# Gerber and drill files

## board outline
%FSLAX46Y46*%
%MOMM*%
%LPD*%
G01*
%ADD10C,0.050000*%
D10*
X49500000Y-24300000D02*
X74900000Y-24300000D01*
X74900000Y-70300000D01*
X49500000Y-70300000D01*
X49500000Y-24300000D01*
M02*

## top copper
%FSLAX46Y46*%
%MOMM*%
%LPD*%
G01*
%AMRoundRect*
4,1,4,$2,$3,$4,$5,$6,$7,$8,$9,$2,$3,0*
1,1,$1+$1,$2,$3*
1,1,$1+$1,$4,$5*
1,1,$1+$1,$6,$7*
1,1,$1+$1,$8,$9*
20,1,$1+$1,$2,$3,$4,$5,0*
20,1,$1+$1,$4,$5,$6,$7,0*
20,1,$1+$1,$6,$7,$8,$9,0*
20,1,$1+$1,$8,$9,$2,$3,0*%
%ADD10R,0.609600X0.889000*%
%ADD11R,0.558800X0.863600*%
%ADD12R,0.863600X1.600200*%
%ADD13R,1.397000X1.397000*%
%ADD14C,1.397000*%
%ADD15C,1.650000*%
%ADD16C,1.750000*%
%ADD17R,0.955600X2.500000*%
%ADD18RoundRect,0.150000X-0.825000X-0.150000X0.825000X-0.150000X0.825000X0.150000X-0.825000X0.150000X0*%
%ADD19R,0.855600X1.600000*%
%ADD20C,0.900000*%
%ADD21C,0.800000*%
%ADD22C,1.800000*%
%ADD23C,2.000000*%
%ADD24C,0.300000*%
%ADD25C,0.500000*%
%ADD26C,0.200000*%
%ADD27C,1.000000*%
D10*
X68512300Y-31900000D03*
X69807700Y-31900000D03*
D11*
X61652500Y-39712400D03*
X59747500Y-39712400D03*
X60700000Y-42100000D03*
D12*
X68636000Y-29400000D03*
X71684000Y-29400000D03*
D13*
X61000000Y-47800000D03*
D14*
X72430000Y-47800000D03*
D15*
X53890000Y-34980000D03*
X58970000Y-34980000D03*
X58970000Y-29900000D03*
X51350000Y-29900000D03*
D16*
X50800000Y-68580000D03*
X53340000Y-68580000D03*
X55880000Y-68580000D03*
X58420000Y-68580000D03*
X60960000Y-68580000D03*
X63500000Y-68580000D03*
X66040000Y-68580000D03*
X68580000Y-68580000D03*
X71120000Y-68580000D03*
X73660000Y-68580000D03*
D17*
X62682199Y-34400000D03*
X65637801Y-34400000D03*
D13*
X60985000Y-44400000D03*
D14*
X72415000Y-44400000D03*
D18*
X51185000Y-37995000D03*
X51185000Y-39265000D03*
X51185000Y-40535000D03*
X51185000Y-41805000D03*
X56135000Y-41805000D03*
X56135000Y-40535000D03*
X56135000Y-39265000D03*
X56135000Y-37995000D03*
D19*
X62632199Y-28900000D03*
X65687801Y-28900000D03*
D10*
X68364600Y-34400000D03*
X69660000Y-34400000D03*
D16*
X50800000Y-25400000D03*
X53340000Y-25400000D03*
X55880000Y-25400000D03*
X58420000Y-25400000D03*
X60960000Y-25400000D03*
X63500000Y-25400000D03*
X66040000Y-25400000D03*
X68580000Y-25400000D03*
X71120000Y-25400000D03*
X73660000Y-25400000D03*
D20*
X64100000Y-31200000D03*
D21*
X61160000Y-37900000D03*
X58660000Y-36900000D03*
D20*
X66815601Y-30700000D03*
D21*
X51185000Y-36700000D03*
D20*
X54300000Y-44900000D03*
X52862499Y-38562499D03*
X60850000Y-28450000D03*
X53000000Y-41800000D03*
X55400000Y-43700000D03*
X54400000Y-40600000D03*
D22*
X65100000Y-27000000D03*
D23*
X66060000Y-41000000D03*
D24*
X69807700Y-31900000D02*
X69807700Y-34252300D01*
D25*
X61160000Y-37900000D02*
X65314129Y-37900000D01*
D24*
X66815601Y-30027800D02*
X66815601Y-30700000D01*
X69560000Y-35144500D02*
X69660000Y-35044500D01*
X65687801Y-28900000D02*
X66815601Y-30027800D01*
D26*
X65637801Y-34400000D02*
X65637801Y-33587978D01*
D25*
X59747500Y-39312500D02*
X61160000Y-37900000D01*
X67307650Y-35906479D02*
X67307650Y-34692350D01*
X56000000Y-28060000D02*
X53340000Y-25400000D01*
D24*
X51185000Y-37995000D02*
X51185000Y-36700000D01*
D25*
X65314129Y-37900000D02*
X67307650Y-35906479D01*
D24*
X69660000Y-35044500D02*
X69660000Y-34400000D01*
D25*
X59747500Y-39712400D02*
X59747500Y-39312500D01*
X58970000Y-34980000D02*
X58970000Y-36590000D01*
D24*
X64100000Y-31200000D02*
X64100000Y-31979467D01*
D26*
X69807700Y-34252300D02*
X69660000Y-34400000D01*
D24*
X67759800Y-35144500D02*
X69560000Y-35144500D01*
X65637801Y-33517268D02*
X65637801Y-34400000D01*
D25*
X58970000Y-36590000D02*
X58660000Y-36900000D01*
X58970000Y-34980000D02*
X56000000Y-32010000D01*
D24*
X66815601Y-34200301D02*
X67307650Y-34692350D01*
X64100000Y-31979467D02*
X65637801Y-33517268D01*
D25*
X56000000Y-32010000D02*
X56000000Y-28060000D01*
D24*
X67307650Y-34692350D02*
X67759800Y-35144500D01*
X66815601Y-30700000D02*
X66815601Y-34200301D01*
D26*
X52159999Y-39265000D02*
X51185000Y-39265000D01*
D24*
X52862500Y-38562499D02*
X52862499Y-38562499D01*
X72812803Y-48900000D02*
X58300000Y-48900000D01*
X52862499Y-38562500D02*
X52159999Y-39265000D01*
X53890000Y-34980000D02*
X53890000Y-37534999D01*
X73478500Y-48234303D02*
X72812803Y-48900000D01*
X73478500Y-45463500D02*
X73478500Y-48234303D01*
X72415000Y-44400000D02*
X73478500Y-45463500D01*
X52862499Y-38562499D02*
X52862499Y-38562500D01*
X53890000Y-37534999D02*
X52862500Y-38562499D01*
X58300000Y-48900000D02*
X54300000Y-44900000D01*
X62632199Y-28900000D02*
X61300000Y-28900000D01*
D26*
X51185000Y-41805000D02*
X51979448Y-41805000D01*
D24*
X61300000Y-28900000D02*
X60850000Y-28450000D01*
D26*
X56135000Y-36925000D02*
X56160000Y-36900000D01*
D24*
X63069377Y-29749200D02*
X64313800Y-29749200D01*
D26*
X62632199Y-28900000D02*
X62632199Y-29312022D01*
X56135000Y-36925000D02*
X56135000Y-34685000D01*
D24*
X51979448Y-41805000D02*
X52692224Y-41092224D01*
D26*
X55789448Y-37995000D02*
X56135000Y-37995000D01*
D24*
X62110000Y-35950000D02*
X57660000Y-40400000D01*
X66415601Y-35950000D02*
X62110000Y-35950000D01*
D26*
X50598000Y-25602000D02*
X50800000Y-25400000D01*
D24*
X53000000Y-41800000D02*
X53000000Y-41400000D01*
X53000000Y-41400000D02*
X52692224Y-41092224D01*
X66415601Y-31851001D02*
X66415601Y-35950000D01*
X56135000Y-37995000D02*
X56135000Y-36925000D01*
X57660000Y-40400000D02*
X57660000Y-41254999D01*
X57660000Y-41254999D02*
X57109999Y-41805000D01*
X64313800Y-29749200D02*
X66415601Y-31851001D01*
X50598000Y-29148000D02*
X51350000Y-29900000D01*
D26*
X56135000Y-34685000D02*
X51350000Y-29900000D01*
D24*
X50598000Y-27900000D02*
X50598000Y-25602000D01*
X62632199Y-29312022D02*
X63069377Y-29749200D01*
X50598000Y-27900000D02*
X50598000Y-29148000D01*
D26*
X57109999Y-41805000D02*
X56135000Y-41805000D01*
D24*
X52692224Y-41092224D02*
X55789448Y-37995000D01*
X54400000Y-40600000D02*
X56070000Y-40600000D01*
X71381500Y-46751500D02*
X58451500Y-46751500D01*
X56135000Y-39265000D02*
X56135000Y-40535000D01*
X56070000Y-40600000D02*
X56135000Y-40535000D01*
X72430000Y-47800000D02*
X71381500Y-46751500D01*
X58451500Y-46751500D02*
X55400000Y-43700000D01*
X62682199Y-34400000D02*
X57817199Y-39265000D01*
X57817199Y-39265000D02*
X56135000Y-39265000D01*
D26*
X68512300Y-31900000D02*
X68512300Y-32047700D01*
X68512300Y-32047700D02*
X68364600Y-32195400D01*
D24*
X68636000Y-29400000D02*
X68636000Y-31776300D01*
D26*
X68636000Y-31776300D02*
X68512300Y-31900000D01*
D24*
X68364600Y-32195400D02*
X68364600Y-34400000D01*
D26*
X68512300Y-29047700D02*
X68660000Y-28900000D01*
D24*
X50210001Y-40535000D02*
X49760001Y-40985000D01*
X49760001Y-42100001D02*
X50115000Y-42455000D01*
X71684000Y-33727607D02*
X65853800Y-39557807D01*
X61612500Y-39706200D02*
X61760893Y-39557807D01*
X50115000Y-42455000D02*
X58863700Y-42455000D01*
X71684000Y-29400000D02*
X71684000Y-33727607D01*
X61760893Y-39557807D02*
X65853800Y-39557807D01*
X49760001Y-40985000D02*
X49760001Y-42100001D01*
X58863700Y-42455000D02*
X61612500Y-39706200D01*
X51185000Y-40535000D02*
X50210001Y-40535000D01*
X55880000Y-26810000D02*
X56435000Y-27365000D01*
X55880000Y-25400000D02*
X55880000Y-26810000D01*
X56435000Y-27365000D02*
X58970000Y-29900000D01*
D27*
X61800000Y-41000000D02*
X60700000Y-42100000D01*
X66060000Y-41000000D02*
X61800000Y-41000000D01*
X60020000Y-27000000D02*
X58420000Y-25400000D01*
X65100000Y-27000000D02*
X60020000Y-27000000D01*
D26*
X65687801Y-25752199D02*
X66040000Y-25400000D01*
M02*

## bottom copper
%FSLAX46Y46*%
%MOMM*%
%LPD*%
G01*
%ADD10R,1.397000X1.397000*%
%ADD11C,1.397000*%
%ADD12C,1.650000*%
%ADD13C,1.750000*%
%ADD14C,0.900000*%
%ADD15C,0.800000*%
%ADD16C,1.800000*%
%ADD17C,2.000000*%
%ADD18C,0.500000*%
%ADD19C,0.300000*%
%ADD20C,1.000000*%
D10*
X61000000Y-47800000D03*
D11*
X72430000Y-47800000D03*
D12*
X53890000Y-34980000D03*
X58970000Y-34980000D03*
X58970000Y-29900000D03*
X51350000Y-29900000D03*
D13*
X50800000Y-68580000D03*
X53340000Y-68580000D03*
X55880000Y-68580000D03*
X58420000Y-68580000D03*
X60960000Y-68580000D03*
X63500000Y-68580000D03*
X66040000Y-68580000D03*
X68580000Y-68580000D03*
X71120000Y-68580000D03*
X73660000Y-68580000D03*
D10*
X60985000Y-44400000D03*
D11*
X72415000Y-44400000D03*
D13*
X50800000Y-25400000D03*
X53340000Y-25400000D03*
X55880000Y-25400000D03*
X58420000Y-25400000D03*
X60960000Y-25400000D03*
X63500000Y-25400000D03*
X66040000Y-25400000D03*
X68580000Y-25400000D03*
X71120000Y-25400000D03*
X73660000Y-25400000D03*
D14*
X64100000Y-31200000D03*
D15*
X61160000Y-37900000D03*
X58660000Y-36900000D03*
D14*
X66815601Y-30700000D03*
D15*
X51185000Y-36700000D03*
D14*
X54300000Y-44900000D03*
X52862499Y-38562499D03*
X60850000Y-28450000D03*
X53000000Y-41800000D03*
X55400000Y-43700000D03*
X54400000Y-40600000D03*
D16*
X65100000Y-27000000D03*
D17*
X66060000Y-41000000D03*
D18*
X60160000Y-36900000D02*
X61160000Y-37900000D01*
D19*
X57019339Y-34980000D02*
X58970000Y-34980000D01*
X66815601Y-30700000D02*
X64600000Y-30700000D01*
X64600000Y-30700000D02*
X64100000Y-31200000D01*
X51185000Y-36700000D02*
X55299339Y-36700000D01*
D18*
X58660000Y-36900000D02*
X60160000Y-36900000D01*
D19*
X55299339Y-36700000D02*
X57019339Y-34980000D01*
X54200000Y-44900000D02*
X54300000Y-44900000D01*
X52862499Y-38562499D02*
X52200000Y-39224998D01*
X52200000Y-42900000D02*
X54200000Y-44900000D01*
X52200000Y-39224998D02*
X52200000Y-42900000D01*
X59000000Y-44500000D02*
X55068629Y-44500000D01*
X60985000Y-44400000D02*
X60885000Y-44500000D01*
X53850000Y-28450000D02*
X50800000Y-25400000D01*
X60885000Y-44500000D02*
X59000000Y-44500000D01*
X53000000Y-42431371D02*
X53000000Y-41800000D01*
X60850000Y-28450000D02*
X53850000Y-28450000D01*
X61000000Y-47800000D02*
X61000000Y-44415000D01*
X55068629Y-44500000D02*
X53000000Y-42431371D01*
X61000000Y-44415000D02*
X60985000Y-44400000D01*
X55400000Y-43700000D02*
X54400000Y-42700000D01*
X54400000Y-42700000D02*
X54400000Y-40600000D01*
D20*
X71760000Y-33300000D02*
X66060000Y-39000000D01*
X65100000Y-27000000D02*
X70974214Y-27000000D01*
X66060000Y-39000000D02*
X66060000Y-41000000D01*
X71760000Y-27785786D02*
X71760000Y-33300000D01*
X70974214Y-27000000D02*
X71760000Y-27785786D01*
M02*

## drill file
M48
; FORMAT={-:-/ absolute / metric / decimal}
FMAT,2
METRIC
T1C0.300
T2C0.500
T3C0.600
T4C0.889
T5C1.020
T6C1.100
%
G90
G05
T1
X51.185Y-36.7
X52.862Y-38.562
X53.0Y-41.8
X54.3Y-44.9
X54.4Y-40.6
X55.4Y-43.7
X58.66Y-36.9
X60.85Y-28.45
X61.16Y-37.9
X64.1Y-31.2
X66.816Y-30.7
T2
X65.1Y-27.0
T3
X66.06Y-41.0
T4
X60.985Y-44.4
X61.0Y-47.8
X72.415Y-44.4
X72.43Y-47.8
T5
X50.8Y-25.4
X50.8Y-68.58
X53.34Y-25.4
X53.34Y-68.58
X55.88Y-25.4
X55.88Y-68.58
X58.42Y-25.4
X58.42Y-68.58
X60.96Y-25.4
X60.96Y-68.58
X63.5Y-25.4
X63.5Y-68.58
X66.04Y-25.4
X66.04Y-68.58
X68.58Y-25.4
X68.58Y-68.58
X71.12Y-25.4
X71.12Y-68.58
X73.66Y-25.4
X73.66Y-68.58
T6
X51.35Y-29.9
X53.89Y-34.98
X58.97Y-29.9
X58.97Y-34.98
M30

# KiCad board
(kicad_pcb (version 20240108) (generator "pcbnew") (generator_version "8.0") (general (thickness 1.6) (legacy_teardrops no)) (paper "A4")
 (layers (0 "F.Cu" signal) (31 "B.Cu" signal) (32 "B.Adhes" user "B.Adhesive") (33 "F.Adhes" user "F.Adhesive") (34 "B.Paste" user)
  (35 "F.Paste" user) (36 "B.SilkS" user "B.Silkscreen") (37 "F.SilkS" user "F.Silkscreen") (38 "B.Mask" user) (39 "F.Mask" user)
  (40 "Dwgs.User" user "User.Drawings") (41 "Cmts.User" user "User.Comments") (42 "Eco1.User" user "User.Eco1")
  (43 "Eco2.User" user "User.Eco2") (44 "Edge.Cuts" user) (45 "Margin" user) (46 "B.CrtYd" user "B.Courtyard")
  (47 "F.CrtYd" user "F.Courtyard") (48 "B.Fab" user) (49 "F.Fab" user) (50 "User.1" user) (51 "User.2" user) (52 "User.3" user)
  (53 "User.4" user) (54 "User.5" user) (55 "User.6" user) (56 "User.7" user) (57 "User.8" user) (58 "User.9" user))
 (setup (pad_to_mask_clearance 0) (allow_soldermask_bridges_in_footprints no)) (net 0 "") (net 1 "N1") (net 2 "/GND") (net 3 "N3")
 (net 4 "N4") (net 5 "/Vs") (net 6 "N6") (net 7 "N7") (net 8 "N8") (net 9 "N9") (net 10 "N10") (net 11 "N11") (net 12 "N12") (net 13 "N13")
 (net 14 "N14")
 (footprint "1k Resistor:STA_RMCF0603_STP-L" (layer "F.Cu") (at 69.16 31.9)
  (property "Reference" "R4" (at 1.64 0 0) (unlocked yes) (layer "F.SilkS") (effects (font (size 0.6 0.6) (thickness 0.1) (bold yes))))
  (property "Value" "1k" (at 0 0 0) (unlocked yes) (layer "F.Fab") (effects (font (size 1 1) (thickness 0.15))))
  (pad "1" smd rect (at -0.6477 0) (size 0.6096 0.889) (layers "F.Cu" "F.Paste" "F.Mask") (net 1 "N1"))
  (pad "2" smd rect (at 0.6477 0) (size 0.6096 0.889) (layers "F.Cu" "F.Paste" "F.Mask") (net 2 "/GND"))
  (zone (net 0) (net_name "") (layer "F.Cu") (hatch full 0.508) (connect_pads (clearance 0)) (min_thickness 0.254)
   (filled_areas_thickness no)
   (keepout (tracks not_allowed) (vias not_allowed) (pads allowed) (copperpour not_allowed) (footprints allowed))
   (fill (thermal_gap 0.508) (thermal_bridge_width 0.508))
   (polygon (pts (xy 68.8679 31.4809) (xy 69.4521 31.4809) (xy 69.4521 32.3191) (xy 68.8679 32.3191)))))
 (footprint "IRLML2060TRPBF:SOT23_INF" (layer "F.Cu") (at 60.7 40.9062 180)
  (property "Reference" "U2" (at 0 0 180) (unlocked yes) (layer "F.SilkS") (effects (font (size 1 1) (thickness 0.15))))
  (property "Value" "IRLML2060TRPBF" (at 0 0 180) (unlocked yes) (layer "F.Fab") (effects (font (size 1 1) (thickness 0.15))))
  (pad "1" smd rect (at -0.9525 1.1938 180) (size 0.5588 0.8636) (layers "F.Cu" "F.Paste" "F.Mask") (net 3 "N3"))
  (pad "2" smd rect (at 0.9525 1.1938 180) (size 0.5588 0.8636) (layers "F.Cu" "F.Paste" "F.Mask") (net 2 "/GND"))
  (pad "3" smd rect (at 0 -1.1938 180) (size 0.5588 0.8636) (layers "F.Cu" "F.Paste" "F.Mask") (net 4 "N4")))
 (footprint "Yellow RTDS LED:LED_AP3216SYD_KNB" (layer "F.Cu") (at 70.16 29.4)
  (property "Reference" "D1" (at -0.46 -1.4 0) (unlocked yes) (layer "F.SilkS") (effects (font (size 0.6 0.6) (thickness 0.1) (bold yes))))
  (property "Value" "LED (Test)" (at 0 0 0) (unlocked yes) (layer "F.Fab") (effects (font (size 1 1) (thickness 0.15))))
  (pad "1" smd rect (at -1.524 0) (size 0.8636 1.6002) (layers "F.Cu" "F.Paste" "F.Mask") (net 1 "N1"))
  (pad "2" smd rect (at 1.524 0) (size 0.8636 1.6002) (layers "F.Cu" "F.Paste" "F.Mask") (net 3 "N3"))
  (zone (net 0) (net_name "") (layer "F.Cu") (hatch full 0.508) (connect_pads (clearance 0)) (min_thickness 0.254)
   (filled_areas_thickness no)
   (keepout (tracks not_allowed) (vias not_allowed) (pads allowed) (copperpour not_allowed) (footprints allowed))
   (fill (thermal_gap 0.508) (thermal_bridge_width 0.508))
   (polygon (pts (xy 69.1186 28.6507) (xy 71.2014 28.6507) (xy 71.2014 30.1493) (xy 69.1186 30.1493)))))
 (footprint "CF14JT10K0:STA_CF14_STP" (layer "F.Cu") (at 61 47.8)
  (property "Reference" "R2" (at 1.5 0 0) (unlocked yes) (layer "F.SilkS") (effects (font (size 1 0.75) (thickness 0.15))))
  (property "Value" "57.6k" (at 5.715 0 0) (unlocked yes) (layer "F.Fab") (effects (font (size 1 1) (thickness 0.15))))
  (pad "1" thru_hole rect (at 0 0) (size 1.397 1.397) (drill 0.889) (layers "*.Cu" "*.Mask") (remove_unused_layers no) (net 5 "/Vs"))
  (pad "2" thru_hole circle (at 11.43 0) (size 1.397 1.397) (drill 0.889) (layers "*.Cu" "*.Mask") (remove_unused_layers no) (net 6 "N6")))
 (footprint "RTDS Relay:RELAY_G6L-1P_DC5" (layer "F.Cu") (at 55.16 32.44)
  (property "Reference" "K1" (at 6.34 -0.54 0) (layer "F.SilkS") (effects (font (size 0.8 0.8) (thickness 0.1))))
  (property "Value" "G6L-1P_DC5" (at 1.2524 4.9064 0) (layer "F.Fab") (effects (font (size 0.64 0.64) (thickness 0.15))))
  (pad "2" thru_hole circle (at -1.27 2.54) (size 1.65 1.65) (drill 1.1) (layers "*.Cu" "*.Mask") (remove_unused_layers no) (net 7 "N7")
   (solder_mask_margin 0.102))
  (pad "4" thru_hole circle (at 3.81 2.54) (size 1.65 1.65) (drill 1.1) (layers "*.Cu" "*.Mask") (remove_unused_layers no) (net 2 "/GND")
   (solder_mask_margin 0.102))
  (pad "5" thru_hole circle (at 3.81 -2.54) (size 1.65 1.65) (drill 1.1) (layers "*.Cu" "*.Mask") (remove_unused_layers no) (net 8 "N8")
   (solder_mask_margin 0.102))
  (pad "8" thru_hole circle (at -3.81 -2.54) (size 1.65 1.65) (drill 1.1) (layers "*.Cu" "*.Mask") (remove_unused_layers no) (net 5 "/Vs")
   (solder_mask_margin 0.102)))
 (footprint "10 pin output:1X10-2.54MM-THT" (layer "F.Cu") (at 50.8 68.58)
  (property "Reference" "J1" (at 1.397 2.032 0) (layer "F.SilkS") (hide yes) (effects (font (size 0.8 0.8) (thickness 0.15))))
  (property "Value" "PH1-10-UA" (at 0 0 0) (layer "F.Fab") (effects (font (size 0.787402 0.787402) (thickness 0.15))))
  (pad "1" thru_hole circle (at 0 0) (size 1.75 1.75) (drill 1.02) (layers "*.Cu" "*.Mask") (remove_unused_layers no)
   (solder_mask_margin 0.102))
  (pad "2" thru_hole circle (at 2.54 0) (size 1.75 1.75) (drill 1.02) (layers "*.Cu" "*.Mask") (remove_unused_layers no)
   (solder_mask_margin 0.102))
  (pad "3" thru_hole circle (at 5.08 0) (size 1.75 1.75) (drill 1.02) (layers "*.Cu" "*.Mask") (remove_unused_layers no)
   (solder_mask_margin 0.102))
  (pad "4" thru_hole circle (at 7.62 0) (size 1.75 1.75) (drill 1.02) (layers "*.Cu" "*.Mask") (remove_unused_layers no)
   (solder_mask_margin 0.102))
  (pad "5" thru_hole circle (at 10.16 0) (size 1.75 1.75) (drill 1.02) (layers "*.Cu" "*.Mask") (remove_unused_layers no)
   (solder_mask_margin 0.102))
  (pad "6" thru_hole circle (at 12.7 0) (size 1.75 1.75) (drill 1.02) (layers "*.Cu" "*.Mask") (remove_unused_layers no)
   (solder_mask_margin 0.102))
  (pad "7" thru_hole circle (at 15.24 0) (size 1.75 1.75) (drill 1.02) (layers "*.Cu" "*.Mask") (remove_unused_layers no)
   (solder_mask_margin 0.102))
  (pad "8" thru_hole circle (at 17.78 0) (size 1.75 1.75) (drill 1.02) (layers "*.Cu" "*.Mask") (remove_unused_layers no)
   (solder_mask_margin 0.102))
  (pad "9" thru_hole circle (at 20.32 0) (size 1.75 1.75) (drill 1.02) (layers "*.Cu" "*.Mask") (remove_unused_layers no)
   (solder_mask_margin 0.102))
  (pad "10" thru_hole circle (at 22.86 0) (size 1.75 1.75) (drill 1.02) (layers "*.Cu" "*.Mask") (remove_unused_layers no)
   (solder_mask_margin 0.102)))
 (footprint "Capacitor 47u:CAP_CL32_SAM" (layer "F.Cu") (at 64.16 34.4)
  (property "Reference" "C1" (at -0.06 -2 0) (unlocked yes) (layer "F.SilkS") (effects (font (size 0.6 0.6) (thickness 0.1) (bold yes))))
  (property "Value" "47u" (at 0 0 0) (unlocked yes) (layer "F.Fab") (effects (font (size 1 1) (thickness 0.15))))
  (pad "1" smd rect (at -1.477801 0) (size 0.9556 2.5) (layers "F.Cu" "F.Paste" "F.Mask") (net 6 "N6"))
  (pad "2" smd rect (at 1.477801 0) (size 0.9556 2.5) (layers "F.Cu" "F.Paste" "F.Mask") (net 2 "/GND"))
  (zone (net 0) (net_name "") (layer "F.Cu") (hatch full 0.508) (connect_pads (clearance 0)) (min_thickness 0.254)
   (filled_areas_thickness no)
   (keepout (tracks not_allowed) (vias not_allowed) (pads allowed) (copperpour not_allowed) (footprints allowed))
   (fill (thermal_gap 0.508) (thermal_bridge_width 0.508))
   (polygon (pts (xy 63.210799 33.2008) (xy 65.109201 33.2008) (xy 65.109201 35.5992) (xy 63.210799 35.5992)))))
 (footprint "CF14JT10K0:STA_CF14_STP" (layer "F.Cu") (at 60.985 44.4)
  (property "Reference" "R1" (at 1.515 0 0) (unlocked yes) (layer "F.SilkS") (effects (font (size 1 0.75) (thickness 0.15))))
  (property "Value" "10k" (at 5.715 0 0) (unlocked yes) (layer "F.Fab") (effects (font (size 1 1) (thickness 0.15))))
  (pad "1" thru_hole rect (at 0 0) (size 1.397 1.397) (drill 0.889) (layers "*.Cu" "*.Mask") (remove_unused_layers no) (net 5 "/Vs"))
  (pad "2" thru_hole circle (at 11.43 0) (size 1.397 1.397) (drill 0.889) (layers "*.Cu" "*.Mask") (remove_unused_layers no) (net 7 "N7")))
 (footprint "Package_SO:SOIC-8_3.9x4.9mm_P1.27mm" (layer "F.Cu") (at 53.66 39.9)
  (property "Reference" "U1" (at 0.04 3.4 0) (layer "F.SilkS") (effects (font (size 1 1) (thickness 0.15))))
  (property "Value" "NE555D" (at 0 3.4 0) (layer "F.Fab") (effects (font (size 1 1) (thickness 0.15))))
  (pad "1" smd roundrect (at -2.475 -1.905) (size 1.95 0.6) (layers "F.Cu" "F.Paste" "F.Mask") (roundrect_rratio 0.25) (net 2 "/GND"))
  (pad "2" smd roundrect (at -2.475 -0.635) (size 1.95 0.6) (layers "F.Cu" "F.Paste" "F.Mask") (roundrect_rratio 0.25) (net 7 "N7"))
  (pad "3" smd roundrect (at -2.475 0.635) (size 1.95 0.6) (layers "F.Cu" "F.Paste" "F.Mask") (roundrect_rratio 0.25) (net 3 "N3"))
  (pad "4" smd roundrect (at -2.475 1.905) (size 1.95 0.6) (layers "F.Cu" "F.Paste" "F.Mask") (roundrect_rratio 0.25) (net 5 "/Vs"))
  (pad "5" smd roundrect (at 2.475 1.905) (size 1.95 0.6) (layers "F.Cu" "F.Paste" "F.Mask") (roundrect_rratio 0.25) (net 5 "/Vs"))
  (pad "6" smd roundrect (at 2.475 0.635) (size 1.95 0.6) (layers "F.Cu" "F.Paste" "F.Mask") (roundrect_rratio 0.25) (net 6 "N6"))
  (pad "7" smd roundrect (at 2.475 -0.635) (size 1.95 0.6) (layers "F.Cu" "F.Paste" "F.Mask") (roundrect_rratio 0.25) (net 6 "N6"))
  (pad "8" smd roundrect (at 2.475 -1.905) (size 1.95 0.6) (layers "F.Cu" "F.Paste" "F.Mask") (roundrect_rratio 0.25) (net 5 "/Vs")))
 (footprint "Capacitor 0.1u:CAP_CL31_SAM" (layer "F.Cu") (at 64.16 28.9)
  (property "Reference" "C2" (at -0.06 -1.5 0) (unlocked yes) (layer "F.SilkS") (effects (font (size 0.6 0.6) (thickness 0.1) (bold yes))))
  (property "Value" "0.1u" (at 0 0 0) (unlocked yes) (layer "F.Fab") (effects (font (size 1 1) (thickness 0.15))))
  (pad "1" smd rect (at -1.527801 0) (size 0.8556 1.6) (layers "F.Cu" "F.Paste" "F.Mask") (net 5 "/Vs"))
  (pad "2" smd rect (at 1.527801 0) (size 0.8556 1.6) (layers "F.Cu" "F.Paste" "F.Mask") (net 2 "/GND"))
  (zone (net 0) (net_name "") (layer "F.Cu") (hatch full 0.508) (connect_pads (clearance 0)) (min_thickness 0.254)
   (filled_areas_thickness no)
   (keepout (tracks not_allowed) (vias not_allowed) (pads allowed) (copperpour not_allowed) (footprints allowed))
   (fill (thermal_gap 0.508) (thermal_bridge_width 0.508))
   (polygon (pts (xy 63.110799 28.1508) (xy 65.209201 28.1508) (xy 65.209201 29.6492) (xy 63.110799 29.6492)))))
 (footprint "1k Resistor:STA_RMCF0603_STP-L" (layer "F.Cu") (at 69.0123 34.4)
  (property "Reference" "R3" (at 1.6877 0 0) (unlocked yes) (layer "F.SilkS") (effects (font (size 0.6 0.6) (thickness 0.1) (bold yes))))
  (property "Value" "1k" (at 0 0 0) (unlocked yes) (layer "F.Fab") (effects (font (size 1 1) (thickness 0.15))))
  (pad "1" smd rect (at -0.6477 0) (size 0.6096 0.889) (layers "F.Cu" "F.Paste" "F.Mask") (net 1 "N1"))
  (pad "2" smd rect (at 0.6477 0) (size 0.6096 0.889) (layers "F.Cu" "F.Paste" "F.Mask") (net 2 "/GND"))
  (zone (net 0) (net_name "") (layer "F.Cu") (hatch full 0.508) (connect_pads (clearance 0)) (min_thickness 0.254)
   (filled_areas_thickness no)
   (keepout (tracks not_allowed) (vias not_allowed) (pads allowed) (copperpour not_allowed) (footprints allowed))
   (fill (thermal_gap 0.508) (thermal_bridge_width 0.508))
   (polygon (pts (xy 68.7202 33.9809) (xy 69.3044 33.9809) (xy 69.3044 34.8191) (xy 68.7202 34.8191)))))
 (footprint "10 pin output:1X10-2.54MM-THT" (layer "F.Cu") (at 50.8 25.4)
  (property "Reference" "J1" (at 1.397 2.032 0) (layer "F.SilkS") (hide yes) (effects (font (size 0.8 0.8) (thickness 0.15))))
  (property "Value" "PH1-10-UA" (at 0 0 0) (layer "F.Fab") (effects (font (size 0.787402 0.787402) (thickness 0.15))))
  (pad "1" thru_hole circle (at 0 0) (size 1.75 1.75) (drill 1.02) (layers "*.Cu" "*.Mask") (remove_unused_layers no) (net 5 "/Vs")
   (solder_mask_margin 0.102))
  (pad "2" thru_hole circle (at 2.54 0) (size 1.75 1.75) (drill 1.02) (layers "*.Cu" "*.Mask") (remove_unused_layers no) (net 2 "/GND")
   (solder_mask_margin 0.102))
  (pad "3" thru_hole circle (at 5.08 0) (size 1.75 1.75) (drill 1.02) (layers "*.Cu" "*.Mask") (remove_unused_layers no) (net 8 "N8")
   (solder_mask_margin 0.102))
  (pad "4" thru_hole circle (at 7.62 0) (size 1.75 1.75) (drill 1.02) (layers "*.Cu" "*.Mask") (remove_unused_layers no) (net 4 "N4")
   (solder_mask_margin 0.102))
  (pad "5" thru_hole circle (at 10.16 0) (size 1.75 1.75) (drill 1.02) (layers "*.Cu" "*.Mask") (remove_unused_layers no) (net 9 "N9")
   (solder_mask_margin 0.102))
  (pad "6" thru_hole circle (at 12.7 0) (size 1.75 1.75) (drill 1.02) (layers "*.Cu" "*.Mask") (remove_unused_layers no) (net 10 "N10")
   (solder_mask_margin 0.102))
  (pad "7" thru_hole circle (at 15.24 0) (size 1.75 1.75) (drill 1.02) (layers "*.Cu" "*.Mask") (remove_unused_layers no) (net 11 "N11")
   (solder_mask_margin 0.102))
  (pad "8" thru_hole circle (at 17.78 0) (size 1.75 1.75) (drill 1.02) (layers "*.Cu" "*.Mask") (remove_unused_layers no) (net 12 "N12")
   (solder_mask_margin 0.102))
  (pad "9" thru_hole circle (at 20.32 0) (size 1.75 1.75) (drill 1.02) (layers "*.Cu" "*.Mask") (remove_unused_layers no) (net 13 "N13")
   (solder_mask_margin 0.102))
  (pad "10" thru_hole circle (at 22.86 0) (size 1.75 1.75) (drill 1.02) (layers "*.Cu" "*.Mask") (remove_unused_layers no) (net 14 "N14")
   (solder_mask_margin 0.102)))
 (gr_rect (start 49.5 24.3) (end 74.9 70.3) (stroke (width 0.05) (type default)) (fill none) (layer "Edge.Cuts"))
 (segment (start 69.8077 31.9) (end 69.8077 34.2523) (width 0.3) (layer "F.Cu") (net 2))
 (segment (start 61.16 37.9) (end 65.314129 37.9) (width 0.5) (layer "F.Cu") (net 2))
 (segment (start 66.815601 30.0278) (end 66.815601 30.7) (width 0.3) (layer "F.Cu") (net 2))
 (segment (start 69.56 35.1445) (end 69.66 35.0445) (width 0.3) (layer "F.Cu") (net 2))
 (segment (start 65.687801 28.9) (end 66.815601 30.0278) (width 0.3) (layer "F.Cu") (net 2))
 (segment (start 65.637801 34.4) (end 65.637801 33.587978) (width 0.2) (layer "F.Cu") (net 2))
 (segment (start 59.7475 39.3125) (end 61.16 37.9) (width 0.5) (layer "F.Cu") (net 2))
 (segment (start 67.30765 35.906479) (end 67.30765 34.69235) (width 0.5) (layer "F.Cu") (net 2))
 (segment (start 56 28.06) (end 53.34 25.4) (width 0.5) (layer "F.Cu") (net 2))
 (segment (start 51.185 37.995) (end 51.185 36.7) (width 0.3) (layer "F.Cu") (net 2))
 (segment (start 65.314129 37.9) (end 67.30765 35.906479) (width 0.5) (layer "F.Cu") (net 2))
 (segment (start 69.66 35.0445) (end 69.66 34.4) (width 0.3) (layer "F.Cu") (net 2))
 (segment (start 59.7475 39.7124) (end 59.7475 39.3125) (width 0.5) (layer "F.Cu") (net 2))
 (segment (start 58.97 34.98) (end 58.97 36.59) (width 0.5) (layer "F.Cu") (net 2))
 (segment (start 64.1 31.2) (end 64.1 31.979467) (width 0.3) (layer "F.Cu") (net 2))
 (segment (start 69.8077 34.2523) (end 69.66 34.4) (width 0.2) (layer "F.Cu") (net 2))
 (segment (start 67.7598 35.1445) (end 69.56 35.1445) (width 0.3) (layer "F.Cu") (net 2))
 (segment (start 65.637801 33.517268) (end 65.637801 34.4) (width 0.3) (layer "F.Cu") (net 2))
 (segment (start 58.97 36.59) (end 58.66 36.9) (width 0.5) (layer "F.Cu") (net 2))
 (segment (start 58.97 34.98) (end 56 32.01) (width 0.5) (layer "F.Cu") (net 2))
 (segment (start 66.815601 34.200301) (end 67.30765 34.69235) (width 0.3) (layer "F.Cu") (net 2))
 (segment (start 64.1 31.979467) (end 65.637801 33.517268) (width 0.3) (layer "F.Cu") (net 2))
 (segment (start 56 32.01) (end 56 28.06) (width 0.5) (layer "F.Cu") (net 2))
 (segment (start 67.30765 34.69235) (end 67.7598 35.1445) (width 0.3) (layer "F.Cu") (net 2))
 (segment (start 66.815601 30.7) (end 66.815601 34.200301) (width 0.3) (layer "F.Cu") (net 2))
 (via (at 64.1 31.2) (size 0.9) (drill 0.3) (layers "F.Cu" "B.Cu") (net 2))
 (via (at 61.16 37.9) (size 0.8) (drill 0.3) (layers "F.Cu" "B.Cu") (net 2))
 (via (at 58.66 36.9) (size 0.8) (drill 0.3) (layers "F.Cu" "B.Cu") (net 2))
 (via (at 66.815601 30.7) (size 0.9) (drill 0.3) (layers "F.Cu" "B.Cu") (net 2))
 (via (at 51.185 36.7) (size 0.8) (drill 0.3) (layers "F.Cu" "B.Cu") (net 2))
 (segment (start 60.16 36.9) (end 61.16 37.9) (width 0.5) (layer "B.Cu") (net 2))
 (segment (start 57.019339 34.98) (end 58.97 34.98) (width 0.3) (layer "B.Cu") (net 2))
 (segment (start 66.815601 30.7) (end 64.6 30.7) (width 0.3) (layer "B.Cu") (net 2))
 (segment (start 64.6 30.7) (end 64.1 31.2) (width 0.3) (layer "B.Cu") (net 2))
 (segment (start 51.185 36.7) (end 55.299339 36.7) (width 0.3) (layer "B.Cu") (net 2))
 (segment (start 58.66 36.9) (end 60.16 36.9) (width 0.5) (layer "B.Cu") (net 2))
 (segment (start 55.299339 36.7) (end 57.019339 34.98) (width 0.3) (layer "B.Cu") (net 2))
 (segment (start 52.159999 39.265) (end 51.185 39.265) (width 0.2) (layer "F.Cu") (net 7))
 (segment (start 52.8625 38.562499) (end 52.862499 38.562499) (width 0.3) (layer "F.Cu") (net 7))
 (segment (start 72.812803 48.9) (end 58.3 48.9) (width 0.3) (layer "F.Cu") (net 7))
 (segment (start 52.862499 38.5625) (end 52.159999 39.265) (width 0.3) (layer "F.Cu") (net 7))
 (segment (start 53.89 34.98) (end 53.89 37.534999) (width 0.3) (layer "F.Cu") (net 7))
 (segment (start 73.4785 48.234303) (end 72.812803 48.9) (width 0.3) (layer "F.Cu") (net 7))
 (segment (start 73.4785 45.4635) (end 73.4785 48.234303) (width 0.3) (layer "F.Cu") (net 7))
 (segment (start 72.415 44.4) (end 73.4785 45.4635) (width 0.3) (layer "F.Cu") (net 7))
 (segment (start 52.862499 38.562499) (end 52.862499 38.5625) (width 0.3) (layer "F.Cu") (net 7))
 (segment (start 53.89 37.534999) (end 52.8625 38.562499) (width 0.3) (layer "F.Cu") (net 7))
 (segment (start 58.3 48.9) (end 54.3 44.9) (width 0.3) (layer "F.Cu") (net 7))
 (via (at 54.3 44.9) (size 0.9) (drill 0.3) (layers "F.Cu" "B.Cu") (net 7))
 (via (at 52.862499 38.562499) (size 0.9) (drill 0.3) (layers "F.Cu" "B.Cu") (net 7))
 (segment (start 54.2 44.9) (end 54.3 44.9) (width 0.3) (layer "B.Cu") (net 7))
 (segment (start 52.862499 38.562499) (end 52.2 39.224998) (width 0.3) (layer "B.Cu") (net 7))
 (segment (start 52.2 42.9) (end 54.2 44.9) (width 0.3) (layer "B.Cu") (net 7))
 (segment (start 52.2 39.224998) (end 52.2 42.9) (width 0.3) (layer "B.Cu") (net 7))
 (segment (start 62.632199 28.9) (end 61.3 28.9) (width 0.3) (layer "F.Cu") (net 5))
 (segment (start 51.185 41.805) (end 51.979448 41.805) (width 0.2) (layer "F.Cu") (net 5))
 (segment (start 61.3 28.9) (end 60.85 28.45) (width 0.3) (layer "F.Cu") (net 5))
 (segment (start 56.135 36.925) (end 56.16 36.9) (width 0.2) (layer "F.Cu") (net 5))
 (segment (start 63.069377 29.7492) (end 64.3138 29.7492) (width 0.3) (layer "F.Cu") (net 5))
 (segment (start 62.632199 28.9) (end 62.632199 29.312022) (width 0.2) (layer "F.Cu") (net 5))
 (segment (start 56.135 36.925) (end 56.135 34.685) (width 0.2) (layer "F.Cu") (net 5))
 (segment (start 51.979448 41.805) (end 52.692224 41.092224) (width 0.3) (layer "F.Cu") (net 5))
 (segment (start 55.789448 37.995) (end 56.135 37.995) (width 0.2) (layer "F.Cu") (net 5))
 (segment (start 62.11 35.95) (end 57.66 40.4) (width 0.3) (layer "F.Cu") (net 5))
 (segment (start 66.415601 35.95) (end 62.11 35.95) (width 0.3) (layer "F.Cu") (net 5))
 (segment (start 50.598 25.602) (end 50.8 25.4) (width 0.2) (layer "F.Cu") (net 5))
 (segment (start 53 41.8) (end 53 41.4) (width 0.3) (layer "F.Cu") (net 5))
 (segment (start 53 41.4) (end 52.692224 41.092224) (width 0.3) (layer "F.Cu") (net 5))
 (segment (start 66.415601 31.851001) (end 66.415601 35.95) (width 0.3) (layer "F.Cu") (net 5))
 (segment (start 56.135 37.995) (end 56.135 36.925) (width 0.3) (layer "F.Cu") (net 5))
 (segment (start 57.66 40.4) (end 57.66 41.254999) (width 0.3) (layer "F.Cu") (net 5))
 (segment (start 57.66 41.254999) (end 57.109999 41.805) (width 0.3) (layer "F.Cu") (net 5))
 (segment (start 64.3138 29.7492) (end 66.415601 31.851001) (width 0.3) (layer "F.Cu") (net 5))
 (segment (start 50.598 29.148) (end 51.35 29.9) (width 0.3) (layer "F.Cu") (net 5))
 (segment (start 56.135 34.685) (end 51.35 29.9) (width 0.2) (layer "F.Cu") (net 5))
 (segment (start 50.598 27.9) (end 50.598 25.602) (width 0.3) (layer "F.Cu") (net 5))
 (segment (start 62.632199 29.312022) (end 63.069377 29.7492) (width 0.3) (layer "F.Cu") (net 5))
 (segment (start 50.598 27.9) (end 50.598 29.148) (width 0.3) (layer "F.Cu") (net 5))
 (segment (start 57.109999 41.805) (end 56.135 41.805) (width 0.2) (layer "F.Cu") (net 5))
 (segment (start 52.692224 41.092224) (end 55.789448 37.995) (width 0.3) (layer "F.Cu") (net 5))
 (via (at 60.85 28.45) (size 0.9) (drill 0.3) (layers "F.Cu" "B.Cu") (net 5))
 (via (at 53 41.8) (size 0.9) (drill 0.3) (layers "F.Cu" "B.Cu") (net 5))
 (segment (start 59 44.5) (end 55.068629 44.5) (width 0.3) (layer "B.Cu") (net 5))
 (segment (start 60.985 44.4) (end 60.885 44.5) (width 0.3) (layer "B.Cu") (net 5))
 (segment (start 53.85 28.45) (end 50.8 25.4) (width 0.3) (layer "B.Cu") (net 5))
 (segment (start 60.885 44.5) (end 59 44.5) (width 0.3) (layer "B.Cu") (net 5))
 (segment (start 53 42.431371) (end 53 41.8) (width 0.3) (layer "B.Cu") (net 5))
 (segment (start 60.85 28.45) (end 53.85 28.45) (width 0.3) (layer "B.Cu") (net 5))
 (segment (start 61 47.8) (end 61 44.415) (width 0.3) (layer "B.Cu") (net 5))
 (segment (start 55.068629 44.5) (end 53 42.431371) (width 0.3) (layer "B.Cu") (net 5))
 (segment (start 61 44.415) (end 60.985 44.4) (width 0.3) (layer "B.Cu") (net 5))
 (segment (start 54.4 40.6) (end 56.07 40.6) (width 0.3) (layer "F.Cu") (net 6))
 (segment (start 71.3815 46.7515) (end 58.4515 46.7515) (width 0.3) (layer "F.Cu") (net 6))
 (segment (start 56.135 39.265) (end 56.135 40.535) (width 0.3) (layer "F.Cu") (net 6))
 (segment (start 56.07 40.6) (end 56.135 40.535) (width 0.3) (layer "F.Cu") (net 6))
 (segment (start 72.43 47.8) (end 71.3815 46.7515) (width 0.3) (layer "F.Cu") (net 6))
 (segment (start 58.4515 46.7515) (end 55.4 43.7) (width 0.3) (layer "F.Cu") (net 6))
 (segment (start 62.682199 34.4) (end 57.817199 39.265) (width 0.3) (layer "F.Cu") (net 6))
 (segment (start 57.817199 39.265) (end 56.135 39.265) (width 0.3) (layer "F.Cu") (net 6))
 (via (at 55.4 43.7) (size 0.9) (drill 0.3) (layers "F.Cu" "B.Cu") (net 6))
 (via (at 54.4 40.6) (size 0.9) (drill 0.3) (layers "F.Cu" "B.Cu") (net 6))
 (segment (start 55.4 43.7) (end 54.4 42.7) (width 0.3) (layer "B.Cu") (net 6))
 (segment (start 54.4 42.7) (end 54.4 40.6) (width 0.3) (layer "B.Cu") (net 6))
 (segment (start 68.5123 31.9) (end 68.5123 32.0477) (width 0.2) (layer "F.Cu") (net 1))
 (segment (start 68.5123 32.0477) (end 68.3646 32.1954) (width 0.2) (layer "F.Cu") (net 1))
 (segment (start 68.636 29.4) (end 68.636 31.7763) (width 0.3) (layer "F.Cu") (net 1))
 (segment (start 68.636 31.7763) (end 68.5123 31.9) (width 0.2) (layer "F.Cu") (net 1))
 (segment (start 68.3646 32.1954) (end 68.3646 34.4) (width 0.3) (layer "F.Cu") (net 1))
 (segment (start 68.5123 29.0477) (end 68.66 28.9) (width 0.2) (layer "F.Cu") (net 1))
 (segment (start 50.210001 40.535) (end 49.760001 40.985) (width 0.3) (layer "F.Cu") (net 3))
 (segment (start 49.760001 42.100001) (end 50.115 42.455) (width 0.3) (layer "F.Cu") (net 3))
 (segment (start 71.684 33.727607) (end 65.8538 39.557807) (width 0.3) (layer "F.Cu") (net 3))
 (segment (start 61.6125 39.7062) (end 61.760893 39.557807) (width 0.3) (layer "F.Cu") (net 3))
 (segment (start 50.115 42.455) (end 58.8637 42.455) (width 0.3) (layer "F.Cu") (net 3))
 (segment (start 71.684 29.4) (end 71.684 33.727607) (width 0.3) (layer "F.Cu") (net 3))
 (segment (start 61.760893 39.557807) (end 65.8538 39.557807) (width 0.3) (layer "F.Cu") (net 3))
 (segment (start 49.760001 40.985) (end 49.760001 42.100001) (width 0.3) (layer "F.Cu") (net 3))
 (segment (start 58.8637 42.455) (end 61.6125 39.7062) (width 0.3) (layer "F.Cu") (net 3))
 (segment (start 51.185 40.535) (end 50.210001 40.535) (width 0.3) (layer "F.Cu") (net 3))
 (segment (start 55.88 26.81) (end 56.435 27.365) (width 0.3) (layer "F.Cu") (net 8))
 (segment (start 55.88 25.4) (end 55.88 26.81) (width 0.3) (layer "F.Cu") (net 8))
 (segment (start 56.435 27.365) (end 58.97 29.9) (width 0.3) (layer "F.Cu") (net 8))
 (segment (start 61.8 41) (end 60.7 42.1) (width 1) (layer "F.Cu") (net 4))
 (segment (start 66.06 41) (end 61.8 41) (width 1) (layer "F.Cu") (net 4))
 (segment (start 60.02 27) (end 58.42 25.4) (width 1) (layer "F.Cu") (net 4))
 (segment (start 65.1 27) (end 60.02 27) (width 1) (layer "F.Cu") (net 4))
 (via (at 65.1 27) (size 1.8) (drill 0.5) (layers "F.Cu" "B.Cu") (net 4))
 (via (at 66.06 41) (size 2) (drill 0.6) (layers "F.Cu" "B.Cu") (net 4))
 (segment (start 71.76 33.3) (end 66.06 39) (width 1) (layer "B.Cu") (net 4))
 (segment (start 65.1 27) (end 70.974214 27) (width 1) (layer "B.Cu") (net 4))
 (segment (start 66.06 39) (end 66.06 41) (width 1) (layer "B.Cu") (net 4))
 (segment (start 71.76 27.785786) (end 71.76 33.3) (width 1) (layer "B.Cu") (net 4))
 (segment (start 70.974214 27) (end 71.76 27.785786) (width 1) (layer "B.Cu") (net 4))
 (segment (start 65.687801 25.752199) (end 66.04 25.4) (width 0.2) (layer "F.Cu") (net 11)))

